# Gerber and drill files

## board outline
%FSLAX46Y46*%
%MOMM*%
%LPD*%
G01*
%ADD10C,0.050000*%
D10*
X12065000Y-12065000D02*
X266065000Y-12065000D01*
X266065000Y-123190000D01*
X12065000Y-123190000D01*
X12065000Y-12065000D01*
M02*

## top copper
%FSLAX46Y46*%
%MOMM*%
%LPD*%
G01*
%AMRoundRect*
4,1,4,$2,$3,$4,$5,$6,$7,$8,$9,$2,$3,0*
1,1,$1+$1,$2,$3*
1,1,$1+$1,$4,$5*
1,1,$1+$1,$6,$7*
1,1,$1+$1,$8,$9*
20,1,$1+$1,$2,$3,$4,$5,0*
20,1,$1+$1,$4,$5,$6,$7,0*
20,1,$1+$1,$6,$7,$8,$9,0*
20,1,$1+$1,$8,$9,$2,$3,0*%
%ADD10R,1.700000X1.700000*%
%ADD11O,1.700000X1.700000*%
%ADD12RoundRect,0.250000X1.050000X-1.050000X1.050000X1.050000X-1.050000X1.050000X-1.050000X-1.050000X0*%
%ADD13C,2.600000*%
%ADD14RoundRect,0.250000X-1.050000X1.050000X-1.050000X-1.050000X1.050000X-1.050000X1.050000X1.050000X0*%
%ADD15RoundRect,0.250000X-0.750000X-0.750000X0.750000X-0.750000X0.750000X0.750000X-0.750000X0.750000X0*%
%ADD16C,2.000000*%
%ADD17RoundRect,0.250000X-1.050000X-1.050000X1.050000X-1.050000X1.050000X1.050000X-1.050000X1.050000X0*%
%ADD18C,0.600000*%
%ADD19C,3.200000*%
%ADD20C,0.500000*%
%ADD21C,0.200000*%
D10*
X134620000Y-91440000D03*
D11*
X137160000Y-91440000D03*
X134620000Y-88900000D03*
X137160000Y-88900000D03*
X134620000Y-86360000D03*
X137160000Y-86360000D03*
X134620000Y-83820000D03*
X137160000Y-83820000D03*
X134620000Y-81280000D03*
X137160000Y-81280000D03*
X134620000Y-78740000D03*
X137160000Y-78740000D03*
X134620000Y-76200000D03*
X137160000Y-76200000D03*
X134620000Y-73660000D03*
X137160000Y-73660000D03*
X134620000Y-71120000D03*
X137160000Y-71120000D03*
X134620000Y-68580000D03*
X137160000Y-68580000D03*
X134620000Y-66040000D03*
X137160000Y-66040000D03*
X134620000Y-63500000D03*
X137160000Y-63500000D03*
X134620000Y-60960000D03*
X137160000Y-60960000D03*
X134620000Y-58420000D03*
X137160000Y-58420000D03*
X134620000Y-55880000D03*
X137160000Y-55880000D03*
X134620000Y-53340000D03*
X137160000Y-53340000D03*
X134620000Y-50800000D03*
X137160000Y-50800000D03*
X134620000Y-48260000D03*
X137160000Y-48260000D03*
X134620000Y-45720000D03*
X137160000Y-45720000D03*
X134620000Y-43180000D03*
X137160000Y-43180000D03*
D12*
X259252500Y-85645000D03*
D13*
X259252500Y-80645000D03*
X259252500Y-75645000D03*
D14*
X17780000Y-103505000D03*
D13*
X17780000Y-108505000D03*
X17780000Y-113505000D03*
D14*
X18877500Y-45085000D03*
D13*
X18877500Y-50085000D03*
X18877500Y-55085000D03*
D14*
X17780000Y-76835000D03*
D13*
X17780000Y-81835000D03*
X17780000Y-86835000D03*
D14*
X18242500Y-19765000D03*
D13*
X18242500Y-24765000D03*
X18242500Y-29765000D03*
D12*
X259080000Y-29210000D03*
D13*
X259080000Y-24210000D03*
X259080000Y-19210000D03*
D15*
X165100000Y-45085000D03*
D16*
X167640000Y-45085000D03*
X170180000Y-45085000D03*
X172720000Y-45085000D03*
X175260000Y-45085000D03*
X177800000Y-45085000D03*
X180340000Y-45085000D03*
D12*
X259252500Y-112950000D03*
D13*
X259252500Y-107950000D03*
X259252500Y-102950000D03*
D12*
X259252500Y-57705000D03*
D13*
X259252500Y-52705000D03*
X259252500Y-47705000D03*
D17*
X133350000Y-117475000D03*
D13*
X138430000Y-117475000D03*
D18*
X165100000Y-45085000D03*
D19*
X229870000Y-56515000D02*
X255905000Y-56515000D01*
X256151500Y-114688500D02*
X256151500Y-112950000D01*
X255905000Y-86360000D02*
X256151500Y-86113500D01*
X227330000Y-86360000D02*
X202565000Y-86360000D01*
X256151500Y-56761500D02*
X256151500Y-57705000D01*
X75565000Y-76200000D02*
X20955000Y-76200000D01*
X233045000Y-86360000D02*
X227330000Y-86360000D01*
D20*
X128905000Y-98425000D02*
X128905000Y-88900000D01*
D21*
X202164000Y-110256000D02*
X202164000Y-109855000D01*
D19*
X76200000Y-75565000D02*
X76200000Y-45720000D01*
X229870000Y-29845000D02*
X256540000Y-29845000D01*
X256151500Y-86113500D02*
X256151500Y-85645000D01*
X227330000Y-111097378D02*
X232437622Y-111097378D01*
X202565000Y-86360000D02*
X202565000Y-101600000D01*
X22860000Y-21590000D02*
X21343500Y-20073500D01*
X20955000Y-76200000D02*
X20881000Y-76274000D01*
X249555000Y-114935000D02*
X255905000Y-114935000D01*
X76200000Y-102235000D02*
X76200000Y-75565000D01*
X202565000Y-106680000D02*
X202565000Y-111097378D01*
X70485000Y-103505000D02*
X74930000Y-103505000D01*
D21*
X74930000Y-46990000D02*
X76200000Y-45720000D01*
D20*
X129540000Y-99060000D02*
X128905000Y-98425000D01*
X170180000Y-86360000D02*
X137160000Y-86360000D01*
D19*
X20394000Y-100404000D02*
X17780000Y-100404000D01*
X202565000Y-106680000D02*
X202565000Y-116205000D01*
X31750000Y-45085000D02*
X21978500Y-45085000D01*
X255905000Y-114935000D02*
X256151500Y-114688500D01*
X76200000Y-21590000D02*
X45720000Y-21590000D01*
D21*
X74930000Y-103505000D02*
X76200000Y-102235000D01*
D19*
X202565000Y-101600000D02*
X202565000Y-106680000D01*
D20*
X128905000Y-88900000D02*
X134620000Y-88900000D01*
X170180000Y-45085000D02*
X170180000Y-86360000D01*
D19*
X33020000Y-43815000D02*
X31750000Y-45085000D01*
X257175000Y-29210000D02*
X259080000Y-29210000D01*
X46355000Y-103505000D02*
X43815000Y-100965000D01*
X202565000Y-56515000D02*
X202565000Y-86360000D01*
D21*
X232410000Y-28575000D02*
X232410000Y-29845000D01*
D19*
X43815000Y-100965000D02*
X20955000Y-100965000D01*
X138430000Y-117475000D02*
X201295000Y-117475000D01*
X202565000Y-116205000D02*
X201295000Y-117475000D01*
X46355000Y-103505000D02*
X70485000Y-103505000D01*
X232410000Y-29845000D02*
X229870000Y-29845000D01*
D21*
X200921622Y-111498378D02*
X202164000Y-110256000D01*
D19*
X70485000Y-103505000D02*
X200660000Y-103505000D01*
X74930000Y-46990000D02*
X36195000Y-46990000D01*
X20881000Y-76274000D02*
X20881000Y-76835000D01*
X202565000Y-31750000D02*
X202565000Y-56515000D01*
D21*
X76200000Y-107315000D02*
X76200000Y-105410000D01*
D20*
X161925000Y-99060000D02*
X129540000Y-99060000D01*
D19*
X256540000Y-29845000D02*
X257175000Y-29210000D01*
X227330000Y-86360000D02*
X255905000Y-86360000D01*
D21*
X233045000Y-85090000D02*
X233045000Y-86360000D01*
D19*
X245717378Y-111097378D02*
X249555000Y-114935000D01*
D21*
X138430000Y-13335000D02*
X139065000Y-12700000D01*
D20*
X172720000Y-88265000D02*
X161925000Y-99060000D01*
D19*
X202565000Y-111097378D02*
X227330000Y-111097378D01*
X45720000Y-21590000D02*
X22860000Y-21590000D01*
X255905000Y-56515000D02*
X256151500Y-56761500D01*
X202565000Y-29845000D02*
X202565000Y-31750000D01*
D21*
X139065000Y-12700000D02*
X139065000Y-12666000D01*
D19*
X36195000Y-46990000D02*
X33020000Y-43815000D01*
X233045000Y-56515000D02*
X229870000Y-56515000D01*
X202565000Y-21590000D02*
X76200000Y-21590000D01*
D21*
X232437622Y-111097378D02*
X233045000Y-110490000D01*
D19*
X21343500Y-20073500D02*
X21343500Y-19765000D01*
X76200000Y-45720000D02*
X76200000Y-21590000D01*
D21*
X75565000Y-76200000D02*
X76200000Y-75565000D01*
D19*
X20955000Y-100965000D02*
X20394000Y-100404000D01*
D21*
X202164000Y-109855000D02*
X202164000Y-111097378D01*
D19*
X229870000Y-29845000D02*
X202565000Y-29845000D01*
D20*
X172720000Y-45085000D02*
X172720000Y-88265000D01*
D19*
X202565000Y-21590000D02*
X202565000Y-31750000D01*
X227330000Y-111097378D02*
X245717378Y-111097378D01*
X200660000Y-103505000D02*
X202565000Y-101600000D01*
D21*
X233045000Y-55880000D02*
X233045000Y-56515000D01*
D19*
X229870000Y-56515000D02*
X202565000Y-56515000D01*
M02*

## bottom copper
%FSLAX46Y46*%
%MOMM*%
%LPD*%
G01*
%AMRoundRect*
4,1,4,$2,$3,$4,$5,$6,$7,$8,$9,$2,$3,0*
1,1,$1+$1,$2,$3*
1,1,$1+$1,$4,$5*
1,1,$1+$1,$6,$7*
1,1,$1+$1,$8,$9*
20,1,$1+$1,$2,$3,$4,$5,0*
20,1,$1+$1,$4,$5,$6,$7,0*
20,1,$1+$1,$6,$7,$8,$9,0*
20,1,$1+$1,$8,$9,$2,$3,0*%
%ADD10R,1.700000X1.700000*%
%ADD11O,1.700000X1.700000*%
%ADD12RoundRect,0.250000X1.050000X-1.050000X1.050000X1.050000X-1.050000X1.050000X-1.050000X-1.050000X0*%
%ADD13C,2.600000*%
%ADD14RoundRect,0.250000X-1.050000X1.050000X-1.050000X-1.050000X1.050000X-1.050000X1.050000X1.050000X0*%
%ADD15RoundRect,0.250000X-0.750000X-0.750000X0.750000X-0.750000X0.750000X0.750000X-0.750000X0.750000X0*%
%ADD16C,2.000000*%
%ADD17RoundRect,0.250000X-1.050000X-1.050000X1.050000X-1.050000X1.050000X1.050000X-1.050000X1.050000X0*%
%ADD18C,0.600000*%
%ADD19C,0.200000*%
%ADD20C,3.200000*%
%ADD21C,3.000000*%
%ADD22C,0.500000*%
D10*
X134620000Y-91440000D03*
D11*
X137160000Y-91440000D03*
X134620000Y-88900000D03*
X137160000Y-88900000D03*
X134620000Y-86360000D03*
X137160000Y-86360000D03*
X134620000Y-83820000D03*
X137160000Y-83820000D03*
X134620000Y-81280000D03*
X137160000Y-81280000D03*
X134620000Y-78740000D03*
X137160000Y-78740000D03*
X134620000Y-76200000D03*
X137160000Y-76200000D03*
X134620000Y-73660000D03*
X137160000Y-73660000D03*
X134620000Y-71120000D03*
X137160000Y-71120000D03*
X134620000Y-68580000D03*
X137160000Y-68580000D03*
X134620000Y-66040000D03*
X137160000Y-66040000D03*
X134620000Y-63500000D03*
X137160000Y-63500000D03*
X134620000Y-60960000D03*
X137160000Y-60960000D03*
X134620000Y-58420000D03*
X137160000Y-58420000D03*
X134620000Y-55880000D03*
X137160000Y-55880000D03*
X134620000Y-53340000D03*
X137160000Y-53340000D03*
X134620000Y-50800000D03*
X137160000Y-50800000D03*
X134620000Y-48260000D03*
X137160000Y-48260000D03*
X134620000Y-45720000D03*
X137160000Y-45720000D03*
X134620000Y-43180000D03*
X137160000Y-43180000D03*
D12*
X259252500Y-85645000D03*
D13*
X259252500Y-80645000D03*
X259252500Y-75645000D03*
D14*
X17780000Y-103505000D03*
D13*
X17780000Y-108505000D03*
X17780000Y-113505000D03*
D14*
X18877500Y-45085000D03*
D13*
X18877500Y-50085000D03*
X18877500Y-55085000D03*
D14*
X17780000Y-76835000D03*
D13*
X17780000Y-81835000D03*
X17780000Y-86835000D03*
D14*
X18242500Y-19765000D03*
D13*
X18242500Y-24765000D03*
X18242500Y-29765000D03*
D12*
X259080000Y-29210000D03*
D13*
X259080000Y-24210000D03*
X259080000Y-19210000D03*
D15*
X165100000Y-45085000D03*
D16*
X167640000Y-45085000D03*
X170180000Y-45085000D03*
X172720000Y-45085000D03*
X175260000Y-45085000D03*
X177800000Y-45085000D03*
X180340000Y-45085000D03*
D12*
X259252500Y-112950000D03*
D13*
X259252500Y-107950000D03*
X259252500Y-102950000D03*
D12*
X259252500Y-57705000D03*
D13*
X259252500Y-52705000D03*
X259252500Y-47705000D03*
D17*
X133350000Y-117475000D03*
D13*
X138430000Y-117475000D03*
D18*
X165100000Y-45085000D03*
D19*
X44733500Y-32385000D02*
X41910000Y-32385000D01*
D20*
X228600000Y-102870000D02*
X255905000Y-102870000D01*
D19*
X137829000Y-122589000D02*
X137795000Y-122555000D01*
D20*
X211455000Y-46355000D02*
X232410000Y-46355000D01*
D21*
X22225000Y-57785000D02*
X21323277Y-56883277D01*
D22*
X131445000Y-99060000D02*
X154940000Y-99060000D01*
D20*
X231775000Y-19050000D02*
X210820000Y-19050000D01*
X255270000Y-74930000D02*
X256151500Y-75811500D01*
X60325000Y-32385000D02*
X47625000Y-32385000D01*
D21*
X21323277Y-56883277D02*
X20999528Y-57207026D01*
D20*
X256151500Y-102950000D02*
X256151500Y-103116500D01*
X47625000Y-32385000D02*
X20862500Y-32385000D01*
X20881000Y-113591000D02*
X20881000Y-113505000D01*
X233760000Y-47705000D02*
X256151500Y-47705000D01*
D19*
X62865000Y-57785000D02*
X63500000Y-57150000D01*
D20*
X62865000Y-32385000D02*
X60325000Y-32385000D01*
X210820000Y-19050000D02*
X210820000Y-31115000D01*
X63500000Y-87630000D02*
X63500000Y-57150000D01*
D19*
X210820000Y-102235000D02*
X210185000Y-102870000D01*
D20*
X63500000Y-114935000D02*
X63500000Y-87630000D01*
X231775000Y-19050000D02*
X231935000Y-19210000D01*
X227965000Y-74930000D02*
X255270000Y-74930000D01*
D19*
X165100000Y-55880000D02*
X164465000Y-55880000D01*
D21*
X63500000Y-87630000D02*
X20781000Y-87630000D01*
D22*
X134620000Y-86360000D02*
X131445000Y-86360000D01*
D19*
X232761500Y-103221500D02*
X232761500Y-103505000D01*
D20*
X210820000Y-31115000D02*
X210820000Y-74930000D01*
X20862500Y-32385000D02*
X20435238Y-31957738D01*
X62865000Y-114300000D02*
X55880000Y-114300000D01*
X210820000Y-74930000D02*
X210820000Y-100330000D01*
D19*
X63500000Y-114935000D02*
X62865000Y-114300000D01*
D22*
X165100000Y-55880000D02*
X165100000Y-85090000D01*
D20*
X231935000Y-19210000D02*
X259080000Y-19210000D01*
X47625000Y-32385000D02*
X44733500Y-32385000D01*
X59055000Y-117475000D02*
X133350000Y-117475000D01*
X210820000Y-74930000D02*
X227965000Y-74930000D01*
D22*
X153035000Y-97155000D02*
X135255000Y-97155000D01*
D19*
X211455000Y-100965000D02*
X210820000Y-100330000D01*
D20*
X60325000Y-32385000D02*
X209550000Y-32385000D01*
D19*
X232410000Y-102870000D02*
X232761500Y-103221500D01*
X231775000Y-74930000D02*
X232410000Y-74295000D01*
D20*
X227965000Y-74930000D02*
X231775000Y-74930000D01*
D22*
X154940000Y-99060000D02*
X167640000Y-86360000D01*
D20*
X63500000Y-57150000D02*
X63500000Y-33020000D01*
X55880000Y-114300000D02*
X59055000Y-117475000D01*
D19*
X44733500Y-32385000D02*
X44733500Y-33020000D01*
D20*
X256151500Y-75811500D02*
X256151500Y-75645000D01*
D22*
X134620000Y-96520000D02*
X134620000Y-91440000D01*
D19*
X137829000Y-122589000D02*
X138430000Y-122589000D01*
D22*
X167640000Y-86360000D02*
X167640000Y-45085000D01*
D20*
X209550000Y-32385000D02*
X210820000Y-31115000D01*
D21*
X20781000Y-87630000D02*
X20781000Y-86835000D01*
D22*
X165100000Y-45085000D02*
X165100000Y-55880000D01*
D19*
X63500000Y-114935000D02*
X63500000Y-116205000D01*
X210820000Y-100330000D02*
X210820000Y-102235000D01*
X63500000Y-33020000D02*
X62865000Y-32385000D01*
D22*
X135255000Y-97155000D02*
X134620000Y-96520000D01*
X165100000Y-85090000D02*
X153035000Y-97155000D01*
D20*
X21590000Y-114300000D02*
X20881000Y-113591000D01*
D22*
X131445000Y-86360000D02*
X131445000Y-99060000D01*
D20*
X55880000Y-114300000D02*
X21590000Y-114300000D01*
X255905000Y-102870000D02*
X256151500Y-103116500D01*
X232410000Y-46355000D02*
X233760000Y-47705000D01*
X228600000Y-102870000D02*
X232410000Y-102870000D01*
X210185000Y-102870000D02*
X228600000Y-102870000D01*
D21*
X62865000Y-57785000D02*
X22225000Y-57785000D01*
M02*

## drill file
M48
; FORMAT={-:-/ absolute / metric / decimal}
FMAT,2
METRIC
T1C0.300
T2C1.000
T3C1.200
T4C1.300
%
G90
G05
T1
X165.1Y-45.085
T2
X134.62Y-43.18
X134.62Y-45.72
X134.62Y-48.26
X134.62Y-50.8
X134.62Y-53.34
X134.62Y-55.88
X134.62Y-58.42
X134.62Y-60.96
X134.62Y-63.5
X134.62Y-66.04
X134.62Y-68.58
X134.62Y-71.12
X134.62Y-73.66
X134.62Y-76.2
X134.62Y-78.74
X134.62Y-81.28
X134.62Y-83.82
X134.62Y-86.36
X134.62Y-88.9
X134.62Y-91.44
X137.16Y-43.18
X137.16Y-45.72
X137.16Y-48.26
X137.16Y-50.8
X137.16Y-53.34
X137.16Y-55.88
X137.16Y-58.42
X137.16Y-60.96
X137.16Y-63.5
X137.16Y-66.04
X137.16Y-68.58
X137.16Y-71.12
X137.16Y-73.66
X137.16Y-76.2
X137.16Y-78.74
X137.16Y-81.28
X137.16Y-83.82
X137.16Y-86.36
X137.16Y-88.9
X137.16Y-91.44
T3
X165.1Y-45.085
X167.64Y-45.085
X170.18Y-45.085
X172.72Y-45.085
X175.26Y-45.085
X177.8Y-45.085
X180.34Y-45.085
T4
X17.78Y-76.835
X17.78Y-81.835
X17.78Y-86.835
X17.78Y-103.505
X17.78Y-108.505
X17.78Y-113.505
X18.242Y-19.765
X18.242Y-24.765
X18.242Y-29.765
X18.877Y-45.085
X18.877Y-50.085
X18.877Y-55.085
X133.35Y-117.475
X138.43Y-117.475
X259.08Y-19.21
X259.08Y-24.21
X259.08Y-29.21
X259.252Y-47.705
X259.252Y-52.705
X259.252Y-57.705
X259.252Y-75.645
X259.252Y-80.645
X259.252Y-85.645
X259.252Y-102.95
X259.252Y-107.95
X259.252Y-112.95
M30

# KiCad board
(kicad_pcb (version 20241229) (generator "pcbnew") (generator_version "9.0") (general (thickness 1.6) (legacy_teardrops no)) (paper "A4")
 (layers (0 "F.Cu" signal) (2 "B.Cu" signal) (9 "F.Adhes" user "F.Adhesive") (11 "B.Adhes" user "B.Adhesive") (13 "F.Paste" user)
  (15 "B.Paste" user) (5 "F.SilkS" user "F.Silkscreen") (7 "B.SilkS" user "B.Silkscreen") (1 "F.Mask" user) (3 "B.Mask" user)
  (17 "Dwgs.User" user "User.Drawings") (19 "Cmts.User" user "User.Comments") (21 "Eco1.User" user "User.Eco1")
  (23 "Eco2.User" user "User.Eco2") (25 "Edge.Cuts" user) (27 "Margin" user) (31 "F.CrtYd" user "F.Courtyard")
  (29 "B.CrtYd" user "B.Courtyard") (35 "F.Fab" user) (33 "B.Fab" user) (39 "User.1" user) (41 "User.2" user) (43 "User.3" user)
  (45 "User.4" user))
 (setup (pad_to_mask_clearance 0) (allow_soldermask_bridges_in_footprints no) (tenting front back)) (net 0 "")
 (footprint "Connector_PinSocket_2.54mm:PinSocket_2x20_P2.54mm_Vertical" (layer "F.Cu") (at 134.62 91.44 180)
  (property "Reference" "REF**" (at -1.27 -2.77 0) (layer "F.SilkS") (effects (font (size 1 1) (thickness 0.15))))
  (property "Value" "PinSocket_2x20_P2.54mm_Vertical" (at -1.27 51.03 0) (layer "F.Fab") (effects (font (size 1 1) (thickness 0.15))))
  (pad "1" thru_hole rect (at 0 0 180) (size 1.7 1.7) (drill 1) (layers "*.Cu" "*.Mask") (remove_unused_layers no))
  (pad "2" thru_hole oval (at -2.54 0 180) (size 1.7 1.7) (drill 1) (layers "*.Cu" "*.Mask") (remove_unused_layers no))
  (pad "3" thru_hole oval (at 0 2.54 180) (size 1.7 1.7) (drill 1) (layers "*.Cu" "*.Mask") (remove_unused_layers no))
  (pad "4" thru_hole oval (at -2.54 2.54 180) (size 1.7 1.7) (drill 1) (layers "*.Cu" "*.Mask") (remove_unused_layers no))
  (pad "5" thru_hole oval (at 0 5.08 180) (size 1.7 1.7) (drill 1) (layers "*.Cu" "*.Mask") (remove_unused_layers no))
  (pad "6" thru_hole oval (at -2.54 5.08 180) (size 1.7 1.7) (drill 1) (layers "*.Cu" "*.Mask") (remove_unused_layers no))
  (pad "7" thru_hole oval (at 0 7.62 180) (size 1.7 1.7) (drill 1) (layers "*.Cu" "*.Mask") (remove_unused_layers no))
  (pad "8" thru_hole oval (at -2.54 7.62 180) (size 1.7 1.7) (drill 1) (layers "*.Cu" "*.Mask") (remove_unused_layers no))
  (pad "9" thru_hole oval (at 0 10.16 180) (size 1.7 1.7) (drill 1) (layers "*.Cu" "*.Mask") (remove_unused_layers no))
  (pad "10" thru_hole oval (at -2.54 10.16 180) (size 1.7 1.7) (drill 1) (layers "*.Cu" "*.Mask") (remove_unused_layers no))
  (pad "11" thru_hole oval (at 0 12.7 180) (size 1.7 1.7) (drill 1) (layers "*.Cu" "*.Mask") (remove_unused_layers no))
  (pad "12" thru_hole oval (at -2.54 12.7 180) (size 1.7 1.7) (drill 1) (layers "*.Cu" "*.Mask") (remove_unused_layers no))
  (pad "13" thru_hole oval (at 0 15.24 180) (size 1.7 1.7) (drill 1) (layers "*.Cu" "*.Mask") (remove_unused_layers no))
  (pad "14" thru_hole oval (at -2.54 15.24 180) (size 1.7 1.7) (drill 1) (layers "*.Cu" "*.Mask") (remove_unused_layers no))
  (pad "15" thru_hole oval (at 0 17.78 180) (size 1.7 1.7) (drill 1) (layers "*.Cu" "*.Mask") (remove_unused_layers no))
  (pad "16" thru_hole oval (at -2.54 17.78 180) (size 1.7 1.7) (drill 1) (layers "*.Cu" "*.Mask") (remove_unused_layers no))
  (pad "17" thru_hole oval (at 0 20.32 180) (size 1.7 1.7) (drill 1) (layers "*.Cu" "*.Mask") (remove_unused_layers no))
  (pad "18" thru_hole oval (at -2.54 20.32 180) (size 1.7 1.7) (drill 1) (layers "*.Cu" "*.Mask") (remove_unused_layers no))
  (pad "19" thru_hole oval (at 0 22.86 180) (size 1.7 1.7) (drill 1) (layers "*.Cu" "*.Mask") (remove_unused_layers no))
  (pad "20" thru_hole oval (at -2.54 22.86 180) (size 1.7 1.7) (drill 1) (layers "*.Cu" "*.Mask") (remove_unused_layers no))
  (pad "21" thru_hole oval (at 0 25.4 180) (size 1.7 1.7) (drill 1) (layers "*.Cu" "*.Mask") (remove_unused_layers no))
  (pad "22" thru_hole oval (at -2.54 25.4 180) (size 1.7 1.7) (drill 1) (layers "*.Cu" "*.Mask") (remove_unused_layers no))
  (pad "23" thru_hole oval (at 0 27.94 180) (size 1.7 1.7) (drill 1) (layers "*.Cu" "*.Mask") (remove_unused_layers no))
  (pad "24" thru_hole oval (at -2.54 27.94 180) (size 1.7 1.7) (drill 1) (layers "*.Cu" "*.Mask") (remove_unused_layers no))
  (pad "25" thru_hole oval (at 0 30.48 180) (size 1.7 1.7) (drill 1) (layers "*.Cu" "*.Mask") (remove_unused_layers no))
  (pad "26" thru_hole oval (at -2.54 30.48 180) (size 1.7 1.7) (drill 1) (layers "*.Cu" "*.Mask") (remove_unused_layers no))
  (pad "27" thru_hole oval (at 0 33.02 180) (size 1.7 1.7) (drill 1) (layers "*.Cu" "*.Mask") (remove_unused_layers no))
  (pad "28" thru_hole oval (at -2.54 33.02 180) (size 1.7 1.7) (drill 1) (layers "*.Cu" "*.Mask") (remove_unused_layers no))
  (pad "29" thru_hole oval (at 0 35.56 180) (size 1.7 1.7) (drill 1) (layers "*.Cu" "*.Mask") (remove_unused_layers no))
  (pad "30" thru_hole oval (at -2.54 35.56 180) (size 1.7 1.7) (drill 1) (layers "*.Cu" "*.Mask") (remove_unused_layers no))
  (pad "31" thru_hole oval (at 0 38.1 180) (size 1.7 1.7) (drill 1) (layers "*.Cu" "*.Mask") (remove_unused_layers no))
  (pad "32" thru_hole oval (at -2.54 38.1 180) (size 1.7 1.7) (drill 1) (layers "*.Cu" "*.Mask") (remove_unused_layers no))
  (pad "33" thru_hole oval (at 0 40.64 180) (size 1.7 1.7) (drill 1) (layers "*.Cu" "*.Mask") (remove_unused_layers no))
  (pad "34" thru_hole oval (at -2.54 40.64 180) (size 1.7 1.7) (drill 1) (layers "*.Cu" "*.Mask") (remove_unused_layers no))
  (pad "35" thru_hole oval (at 0 43.18 180) (size 1.7 1.7) (drill 1) (layers "*.Cu" "*.Mask") (remove_unused_layers no))
  (pad "36" thru_hole oval (at -2.54 43.18 180) (size 1.7 1.7) (drill 1) (layers "*.Cu" "*.Mask") (remove_unused_layers no))
  (pad "37" thru_hole oval (at 0 45.72 180) (size 1.7 1.7) (drill 1) (layers "*.Cu" "*.Mask") (remove_unused_layers no))
  (pad "38" thru_hole oval (at -2.54 45.72 180) (size 1.7 1.7) (drill 1) (layers "*.Cu" "*.Mask") (remove_unused_layers no))
  (pad "39" thru_hole oval (at 0 48.26 180) (size 1.7 1.7) (drill 1) (layers "*.Cu" "*.Mask") (remove_unused_layers no))
  (pad "40" thru_hole oval (at -2.54 48.26 180) (size 1.7 1.7) (drill 1) (layers "*.Cu" "*.Mask") (remove_unused_layers no)))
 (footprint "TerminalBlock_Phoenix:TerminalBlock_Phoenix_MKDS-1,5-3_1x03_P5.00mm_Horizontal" (layer "F.Cu") (at 259.2525 85.645 90)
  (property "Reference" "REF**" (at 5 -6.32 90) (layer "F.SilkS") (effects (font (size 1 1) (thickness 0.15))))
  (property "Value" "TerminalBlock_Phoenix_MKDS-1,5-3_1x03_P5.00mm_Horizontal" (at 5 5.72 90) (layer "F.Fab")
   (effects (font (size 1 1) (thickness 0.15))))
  (pad "1" thru_hole roundrect (at 0 0 90) (size 2.6 2.6) (drill 1.3) (layers "*.Cu" "*.Mask") (remove_unused_layers no)
   (roundrect_rratio 0.096154))
  (pad "2" thru_hole circle (at 5 0 90) (size 2.6 2.6) (drill 1.3) (layers "*.Cu" "*.Mask") (remove_unused_layers no))
  (pad "3" thru_hole circle (at 10 0 90) (size 2.6 2.6) (drill 1.3) (layers "*.Cu" "*.Mask") (remove_unused_layers no)))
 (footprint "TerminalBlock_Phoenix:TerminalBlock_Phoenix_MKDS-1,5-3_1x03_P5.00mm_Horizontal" (layer "F.Cu") (at 17.78 103.505 -90)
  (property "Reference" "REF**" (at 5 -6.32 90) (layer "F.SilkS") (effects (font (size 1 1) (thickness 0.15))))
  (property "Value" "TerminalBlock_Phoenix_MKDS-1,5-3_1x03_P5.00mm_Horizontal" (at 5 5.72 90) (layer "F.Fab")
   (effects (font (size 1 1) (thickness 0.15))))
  (pad "1" thru_hole roundrect (at 0 0 270) (size 2.6 2.6) (drill 1.3) (layers "*.Cu" "*.Mask") (remove_unused_layers no)
   (roundrect_rratio 0.096154))
  (pad "2" thru_hole circle (at 5 0 270) (size 2.6 2.6) (drill 1.3) (layers "*.Cu" "*.Mask") (remove_unused_layers no))
  (pad "3" thru_hole circle (at 10 0 270) (size 2.6 2.6) (drill 1.3) (layers "*.Cu" "*.Mask") (remove_unused_layers no)))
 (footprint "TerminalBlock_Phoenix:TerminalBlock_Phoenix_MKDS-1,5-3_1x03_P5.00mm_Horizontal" (layer "F.Cu") (at 18.8775 45.085 -90)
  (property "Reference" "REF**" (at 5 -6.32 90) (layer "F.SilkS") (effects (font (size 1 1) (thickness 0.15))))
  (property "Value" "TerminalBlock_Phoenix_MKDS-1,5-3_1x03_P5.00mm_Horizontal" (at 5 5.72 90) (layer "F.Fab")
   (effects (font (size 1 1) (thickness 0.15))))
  (pad "1" thru_hole roundrect (at 0 0 270) (size 2.6 2.6) (drill 1.3) (layers "*.Cu" "*.Mask") (remove_unused_layers no)
   (roundrect_rratio 0.096154))
  (pad "2" thru_hole circle (at 5 0 270) (size 2.6 2.6) (drill 1.3) (layers "*.Cu" "*.Mask") (remove_unused_layers no))
  (pad "3" thru_hole circle (at 10 0 270) (size 2.6 2.6) (drill 1.3) (layers "*.Cu" "*.Mask") (remove_unused_layers no)))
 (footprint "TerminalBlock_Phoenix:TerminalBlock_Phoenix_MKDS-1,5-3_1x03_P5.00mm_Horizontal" (layer "F.Cu") (at 17.78 76.835 -90)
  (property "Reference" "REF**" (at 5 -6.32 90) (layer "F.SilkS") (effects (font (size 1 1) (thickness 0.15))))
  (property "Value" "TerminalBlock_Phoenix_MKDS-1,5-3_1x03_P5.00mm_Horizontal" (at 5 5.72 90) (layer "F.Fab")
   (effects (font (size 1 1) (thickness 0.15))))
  (pad "1" thru_hole roundrect (at 0 0 270) (size 2.6 2.6) (drill 1.3) (layers "*.Cu" "*.Mask") (remove_unused_layers no)
   (roundrect_rratio 0.096154))
  (pad "2" thru_hole circle (at 5 0 270) (size 2.6 2.6) (drill 1.3) (layers "*.Cu" "*.Mask") (remove_unused_layers no))
  (pad "3" thru_hole circle (at 10 0 270) (size 2.6 2.6) (drill 1.3) (layers "*.Cu" "*.Mask") (remove_unused_layers no)))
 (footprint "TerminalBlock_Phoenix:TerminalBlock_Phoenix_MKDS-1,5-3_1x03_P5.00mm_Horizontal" (layer "F.Cu") (at 18.2425 19.765 -90)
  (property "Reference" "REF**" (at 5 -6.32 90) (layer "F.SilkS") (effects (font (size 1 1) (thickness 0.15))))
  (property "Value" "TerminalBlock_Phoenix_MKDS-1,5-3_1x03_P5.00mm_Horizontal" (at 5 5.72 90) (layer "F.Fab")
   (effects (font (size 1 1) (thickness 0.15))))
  (pad "1" thru_hole roundrect (at 0 0 270) (size 2.6 2.6) (drill 1.3) (layers "*.Cu" "*.Mask") (remove_unused_layers no)
   (roundrect_rratio 0.096154))
  (pad "2" thru_hole circle (at 5 0 270) (size 2.6 2.6) (drill 1.3) (layers "*.Cu" "*.Mask") (remove_unused_layers no))
  (pad "3" thru_hole circle (at 10 0 270) (size 2.6 2.6) (drill 1.3) (layers "*.Cu" "*.Mask") (remove_unused_layers no)))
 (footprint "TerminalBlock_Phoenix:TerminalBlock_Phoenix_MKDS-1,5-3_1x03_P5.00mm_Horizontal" (layer "F.Cu") (at 259.08 29.21 90)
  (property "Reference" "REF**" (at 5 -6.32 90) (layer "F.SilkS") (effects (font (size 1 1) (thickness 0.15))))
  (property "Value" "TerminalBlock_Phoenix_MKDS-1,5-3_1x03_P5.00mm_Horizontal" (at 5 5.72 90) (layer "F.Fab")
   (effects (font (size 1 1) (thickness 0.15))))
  (pad "1" thru_hole roundrect (at 0 0 90) (size 2.6 2.6) (drill 1.3) (layers "*.Cu" "*.Mask") (remove_unused_layers no)
   (roundrect_rratio 0.096154))
  (pad "2" thru_hole circle (at 5 0 90) (size 2.6 2.6) (drill 1.3) (layers "*.Cu" "*.Mask") (remove_unused_layers no))
  (pad "3" thru_hole circle (at 10 0 90) (size 2.6 2.6) (drill 1.3) (layers "*.Cu" "*.Mask") (remove_unused_layers no)))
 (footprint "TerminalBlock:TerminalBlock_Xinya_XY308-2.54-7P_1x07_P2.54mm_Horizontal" (layer "F.Cu") (at 165.1 45.085)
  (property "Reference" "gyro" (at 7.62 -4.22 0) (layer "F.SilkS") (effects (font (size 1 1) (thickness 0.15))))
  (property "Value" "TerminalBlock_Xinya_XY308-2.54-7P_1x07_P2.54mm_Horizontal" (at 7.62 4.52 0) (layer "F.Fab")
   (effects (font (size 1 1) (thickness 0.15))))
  (pad "1" thru_hole roundrect (at 0 0) (size 2 2) (drill 1.2) (layers "*.Cu" "*.Mask") (remove_unused_layers no) (roundrect_rratio 0.125))
  (pad "2" thru_hole circle (at 2.54 0) (size 2 2) (drill 1.2) (layers "*.Cu" "*.Mask") (remove_unused_layers no))
  (pad "3" thru_hole circle (at 5.08 0) (size 2 2) (drill 1.2) (layers "*.Cu" "*.Mask") (remove_unused_layers no))
  (pad "4" thru_hole circle (at 7.62 0) (size 2 2) (drill 1.2) (layers "*.Cu" "*.Mask") (remove_unused_layers no))
  (pad "5" thru_hole circle (at 10.16 0) (size 2 2) (drill 1.2) (layers "*.Cu" "*.Mask") (remove_unused_layers no))
  (pad "6" thru_hole circle (at 12.7 0) (size 2 2) (drill 1.2) (layers "*.Cu" "*.Mask") (remove_unused_layers no))
  (pad "7" thru_hole circle (at 15.24 0) (size 2 2) (drill 1.2) (layers "*.Cu" "*.Mask") (remove_unused_layers no)))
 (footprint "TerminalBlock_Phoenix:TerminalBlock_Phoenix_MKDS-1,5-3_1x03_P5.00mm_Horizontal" (layer "F.Cu") (at 259.2525 112.95 90)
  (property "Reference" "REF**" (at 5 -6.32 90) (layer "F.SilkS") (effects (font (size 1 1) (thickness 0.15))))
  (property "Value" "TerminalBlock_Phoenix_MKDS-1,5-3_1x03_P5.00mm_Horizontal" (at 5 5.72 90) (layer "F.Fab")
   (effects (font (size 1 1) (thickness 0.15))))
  (pad "1" thru_hole roundrect (at 0 0 90) (size 2.6 2.6) (drill 1.3) (layers "*.Cu" "*.Mask") (remove_unused_layers no)
   (roundrect_rratio 0.096154))
  (pad "2" thru_hole circle (at 5 0 90) (size 2.6 2.6) (drill 1.3) (layers "*.Cu" "*.Mask") (remove_unused_layers no))
  (pad "3" thru_hole circle (at 10 0 90) (size 2.6 2.6) (drill 1.3) (layers "*.Cu" "*.Mask") (remove_unused_layers no)))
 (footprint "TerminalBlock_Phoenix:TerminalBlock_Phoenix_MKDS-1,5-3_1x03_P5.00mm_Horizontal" (layer "F.Cu") (at 259.2525 57.705 90)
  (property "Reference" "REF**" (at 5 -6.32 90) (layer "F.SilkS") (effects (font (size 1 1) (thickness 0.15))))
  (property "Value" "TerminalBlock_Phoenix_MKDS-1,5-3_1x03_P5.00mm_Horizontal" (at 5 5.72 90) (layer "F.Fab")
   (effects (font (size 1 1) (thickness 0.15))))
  (pad "1" thru_hole roundrect (at 0 0 90) (size 2.6 2.6) (drill 1.3) (layers "*.Cu" "*.Mask") (remove_unused_layers no)
   (roundrect_rratio 0.096154))
  (pad "2" thru_hole circle (at 5 0 90) (size 2.6 2.6) (drill 1.3) (layers "*.Cu" "*.Mask") (remove_unused_layers no))
  (pad "3" thru_hole circle (at 10 0 90) (size 2.6 2.6) (drill 1.3) (layers "*.Cu" "*.Mask") (remove_unused_layers no)))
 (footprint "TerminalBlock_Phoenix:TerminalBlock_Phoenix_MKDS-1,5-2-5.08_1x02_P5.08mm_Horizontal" (layer "F.Cu") (at 133.35 117.475)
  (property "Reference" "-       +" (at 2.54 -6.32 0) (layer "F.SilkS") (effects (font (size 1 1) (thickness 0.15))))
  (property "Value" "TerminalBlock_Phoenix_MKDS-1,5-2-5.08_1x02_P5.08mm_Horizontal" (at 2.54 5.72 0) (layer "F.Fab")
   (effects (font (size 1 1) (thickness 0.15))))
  (pad "1" thru_hole roundrect (at 0 0) (size 2.6 2.6) (drill 1.3) (layers "*.Cu" "*.Mask") (remove_unused_layers no)
   (roundrect_rratio 0.096154))
  (pad "2" thru_hole circle (at 5.08 0) (size 2.6 2.6) (drill 1.3) (layers "*.Cu" "*.Mask") (remove_unused_layers no)))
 (gr_rect (start 12.065 12.065) (end 266.065 123.19) (stroke (width 0.05) (type default)) (fill no) (layer "Edge.Cuts"))
 (segment (start 229.87 56.515) (end 255.905 56.515) (width 3.2) (layer "F.Cu") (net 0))
 (segment (start 256.1515 114.6885) (end 256.1515 112.95) (width 3.2) (layer "F.Cu") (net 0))
 (segment (start 255.905 86.36) (end 256.1515 86.1135) (width 3.2) (layer "F.Cu") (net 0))
 (segment (start 227.33 86.36) (end 202.565 86.36) (width 3.2) (layer "F.Cu") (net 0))
 (segment (start 256.1515 56.7615) (end 256.1515 57.705) (width 3.2) (layer "F.Cu") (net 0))
 (segment (start 75.565 76.2) (end 20.955 76.2) (width 3.2) (layer "F.Cu") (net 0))
 (segment (start 233.045 86.36) (end 227.33 86.36) (width 3.2) (layer "F.Cu") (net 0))
 (segment (start 128.905 98.425) (end 128.905 88.9) (width 0.5) (layer "F.Cu") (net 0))
 (segment (start 202.164 110.256) (end 202.164 109.855) (width 0.2) (layer "F.Cu") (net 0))
 (segment (start 76.2 75.565) (end 76.2 45.72) (width 3.2) (layer "F.Cu") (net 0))
 (segment (start 229.87 29.845) (end 256.54 29.845) (width 3.2) (layer "F.Cu") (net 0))
 (segment (start 256.1515 86.1135) (end 256.1515 85.645) (width 3.2) (layer "F.Cu") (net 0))
 (segment (start 227.33 111.097378) (end 232.437622 111.097378) (width 3.2) (layer "F.Cu") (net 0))
 (segment (start 202.565 86.36) (end 202.565 101.6) (width 3.2) (layer "F.Cu") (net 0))
 (segment (start 22.86 21.59) (end 21.3435 20.0735) (width 3.2) (layer "F.Cu") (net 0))
 (segment (start 20.955 76.2) (end 20.881 76.274) (width 3.2) (layer "F.Cu") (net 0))
 (segment (start 249.555 114.935) (end 255.905 114.935) (width 3.2) (layer "F.Cu") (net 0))
 (segment (start 76.2 102.235) (end 76.2 75.565) (width 3.2) (layer "F.Cu") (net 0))
 (segment (start 202.565 106.68) (end 202.565 111.097378) (width 3.2) (layer "F.Cu") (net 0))
 (segment (start 70.485 103.505) (end 74.93 103.505) (width 3.2) (layer "F.Cu") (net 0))
 (segment (start 74.93 46.99) (end 76.2 45.72) (width 0.2) (layer "F.Cu") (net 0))
 (segment (start 129.54 99.06) (end 128.905 98.425) (width 0.5) (layer "F.Cu") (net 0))
 (segment (start 170.18 86.36) (end 137.16 86.36) (width 0.5) (layer "F.Cu") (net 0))
 (segment (start 20.394 100.404) (end 17.78 100.404) (width 3.2) (layer "F.Cu") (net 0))
 (segment (start 202.565 106.68) (end 202.565 116.205) (width 3.2) (layer "F.Cu") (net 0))
 (segment (start 31.75 45.085) (end 21.9785 45.085) (width 3.2) (layer "F.Cu") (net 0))
 (segment (start 255.905 114.935) (end 256.1515 114.6885) (width 3.2) (layer "F.Cu") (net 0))
 (segment (start 76.2 21.59) (end 45.72 21.59) (width 3.2) (layer "F.Cu") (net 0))
 (segment (start 74.93 103.505) (end 76.2 102.235) (width 0.2) (layer "F.Cu") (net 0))
 (segment (start 202.565 101.6) (end 202.565 106.68) (width 3.2) (layer "F.Cu") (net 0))
 (segment (start 128.905 88.9) (end 134.62 88.9) (width 0.5) (layer "F.Cu") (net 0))
 (segment (start 170.18 45.085) (end 170.18 86.36) (width 0.5) (layer "F.Cu") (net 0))
 (segment (start 33.02 43.815) (end 31.75 45.085) (width 3.2) (layer "F.Cu") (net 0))
 (segment (start 257.175 29.21) (end 259.08 29.21) (width 3.2) (layer "F.Cu") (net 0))
 (segment (start 46.355 103.505) (end 43.815 100.965) (width 3.2) (layer "F.Cu") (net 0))
 (segment (start 202.565 56.515) (end 202.565 86.36) (width 3.2) (layer "F.Cu") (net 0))
 (segment (start 232.41 28.575) (end 232.41 29.845) (width 0.2) (layer "F.Cu") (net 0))
 (segment (start 43.815 100.965) (end 20.955 100.965) (width 3.2) (layer "F.Cu") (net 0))
 (segment (start 138.43 117.475) (end 201.295 117.475) (width 3.2) (layer "F.Cu") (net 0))
 (segment (start 202.565 116.205) (end 201.295 117.475) (width 3.2) (layer "F.Cu") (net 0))
 (segment (start 46.355 103.505) (end 70.485 103.505) (width 3.2) (layer "F.Cu") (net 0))
 (segment (start 232.41 29.845) (end 229.87 29.845) (width 3.2) (layer "F.Cu") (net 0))
 (segment (start 200.921622 111.498378) (end 202.164 110.256) (width 0.2) (layer "F.Cu") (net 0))
 (segment (start 70.485 103.505) (end 200.66 103.505) (width 3.2) (layer "F.Cu") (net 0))
 (segment (start 74.93 46.99) (end 36.195 46.99) (width 3.2) (layer "F.Cu") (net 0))
 (segment (start 20.881 76.274) (end 20.881 76.835) (width 3.2) (layer "F.Cu") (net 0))
 (segment (start 202.565 31.75) (end 202.565 56.515) (width 3.2) (layer "F.Cu") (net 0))
 (segment (start 76.2 107.315) (end 76.2 105.41) (width 0.2) (layer "F.Cu") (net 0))
 (segment (start 161.925 99.06) (end 129.54 99.06) (width 0.5) (layer "F.Cu") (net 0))
 (segment (start 256.54 29.845) (end 257.175 29.21) (width 3.2) (layer "F.Cu") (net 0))
 (segment (start 227.33 86.36) (end 255.905 86.36) (width 3.2) (layer "F.Cu") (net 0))
 (segment (start 233.045 85.09) (end 233.045 86.36) (width 0.2) (layer "F.Cu") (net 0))
 (segment (start 245.717378 111.097378) (end 249.555 114.935) (width 3.2) (layer "F.Cu") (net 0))
 (segment (start 138.43 13.335) (end 139.065 12.7) (width 0.2) (layer "F.Cu") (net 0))
 (segment (start 172.72 88.265) (end 161.925 99.06) (width 0.5) (layer "F.Cu") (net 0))
 (segment (start 202.565 111.097378) (end 227.33 111.097378) (width 3.2) (layer "F.Cu") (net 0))
 (segment (start 45.72 21.59) (end 22.86 21.59) (width 3.2) (layer "F.Cu") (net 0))
 (segment (start 255.905 56.515) (end 256.1515 56.7615) (width 3.2) (layer "F.Cu") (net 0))
 (segment (start 202.565 29.845) (end 202.565 31.75) (width 3.2) (layer "F.Cu") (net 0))
 (segment (start 139.065 12.7) (end 139.065 12.666) (width 0.2) (layer "F.Cu") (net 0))
 (segment (start 36.195 46.99) (end 33.02 43.815) (width 3.2) (layer "F.Cu") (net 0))
 (segment (start 233.045 56.515) (end 229.87 56.515) (width 3.2) (layer "F.Cu") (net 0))
 (segment (start 202.565 21.59) (end 76.2 21.59) (width 3.2) (layer "F.Cu") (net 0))
 (segment (start 232.437622 111.097378) (end 233.045 110.49) (width 0.2) (layer "F.Cu") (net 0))
 (segment (start 21.3435 20.0735) (end 21.3435 19.765) (width 3.2) (layer "F.Cu") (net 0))
 (segment (start 76.2 45.72) (end 76.2 21.59) (width 3.2) (layer "F.Cu") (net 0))
 (segment (start 75.565 76.2) (end 76.2 75.565) (width 0.2) (layer "F.Cu") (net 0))
 (segment (start 20.955 100.965) (end 20.394 100.404) (width 3.2) (layer "F.Cu") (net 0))
 (segment (start 202.164 109.855) (end 202.164 111.097378) (width 0.2) (layer "F.Cu") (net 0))
 (segment (start 229.87 29.845) (end 202.565 29.845) (width 3.2) (layer "F.Cu") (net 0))
 (segment (start 172.72 45.085) (end 172.72 88.265) (width 0.5) (layer "F.Cu") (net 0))
 (segment (start 202.565 21.59) (end 202.565 31.75) (width 3.2) (layer "F.Cu") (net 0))
 (segment (start 227.33 111.097378) (end 245.717378 111.097378) (width 3.2) (layer "F.Cu") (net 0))
 (segment (start 200.66 103.505) (end 202.565 101.6) (width 3.2) (layer "F.Cu") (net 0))
 (segment (start 233.045 55.88) (end 233.045 56.515) (width 0.2) (layer "F.Cu") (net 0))
 (segment (start 229.87 56.515) (end 202.565 56.515) (width 3.2) (layer "F.Cu") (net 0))
 (via (at 165.1 45.085) (size 0.6) (drill 0.3) (layers "F.Cu" "B.Cu") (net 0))
 (segment (start 44.7335 32.385) (end 41.91 32.385) (width 0.2) (layer "B.Cu") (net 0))
 (segment (start 228.6 102.87) (end 255.905 102.87) (width 3.2) (layer "B.Cu") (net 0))
 (segment (start 137.829 122.589) (end 137.795 122.555) (width 0.2) (layer "B.Cu") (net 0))
 (segment (start 211.455 46.355) (end 232.41 46.355) (width 3.2) (layer "B.Cu") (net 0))
 (segment (start 22.225 57.785) (end 21.323277 56.883277) (width 3) (layer "B.Cu") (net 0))
 (segment (start 131.445 99.06) (end 154.94 99.06) (width 0.5) (layer "B.Cu") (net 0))
 (segment (start 231.775 19.05) (end 210.82 19.05) (width 3.2) (layer "B.Cu") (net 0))
 (segment (start 255.27 74.93) (end 256.1515 75.8115) (width 3.2) (layer "B.Cu") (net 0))
 (segment (start 60.325 32.385) (end 47.625 32.385) (width 3.2) (layer "B.Cu") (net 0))
 (segment (start 21.323277 56.883277) (end 20.999528 57.207026) (width 3) (layer "B.Cu") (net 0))
 (segment (start 256.1515 102.95) (end 256.1515 103.1165) (width 3.2) (layer "B.Cu") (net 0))
 (segment (start 47.625 32.385) (end 20.8625 32.385) (width 3.2) (layer "B.Cu") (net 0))
 (segment (start 20.881 113.591) (end 20.881 113.505) (width 3.2) (layer "B.Cu") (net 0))
 (segment (start 233.76 47.705) (end 256.1515 47.705) (width 3.2) (layer "B.Cu") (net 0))
 (segment (start 62.865 57.785) (end 63.5 57.15) (width 0.2) (layer "B.Cu") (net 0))
 (segment (start 62.865 32.385) (end 60.325 32.385) (width 3.2) (layer "B.Cu") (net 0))
 (segment (start 210.82 19.05) (end 210.82 31.115) (width 3.2) (layer "B.Cu") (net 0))
 (segment (start 63.5 87.63) (end 63.5 57.15) (width 3.2) (layer "B.Cu") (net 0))
 (segment (start 210.82 102.235) (end 210.185 102.87) (width 0.2) (layer "B.Cu") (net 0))
 (segment (start 63.5 114.935) (end 63.5 87.63) (width 3.2) (layer "B.Cu") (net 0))
 (segment (start 231.775 19.05) (end 231.935 19.21) (width 3.2) (layer "B.Cu") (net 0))
 (segment (start 227.965 74.93) (end 255.27 74.93) (width 3.2) (layer "B.Cu") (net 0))
 (segment (start 165.1 55.88) (end 164.465 55.88) (width 0.2) (layer "B.Cu") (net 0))
 (segment (start 63.5 87.63) (end 20.781 87.63) (width 3) (layer "B.Cu") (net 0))
 (segment (start 134.62 86.36) (end 131.445 86.36) (width 0.5) (layer "B.Cu") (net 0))
 (segment (start 232.7615 103.2215) (end 232.7615 103.505) (width 0.2) (layer "B.Cu") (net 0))
 (segment (start 210.82 31.115) (end 210.82 74.93) (width 3.2) (layer "B.Cu") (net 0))
 (segment (start 20.8625 32.385) (end 20.435238 31.957738) (width 3.2) (layer "B.Cu") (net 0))
 (segment (start 62.865 114.3) (end 55.88 114.3) (width 3.2) (layer "B.Cu") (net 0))
 (segment (start 210.82 74.93) (end 210.82 100.33) (width 3.2) (layer "B.Cu") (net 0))
 (segment (start 63.5 114.935) (end 62.865 114.3) (width 0.2) (layer "B.Cu") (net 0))
 (segment (start 165.1 55.88) (end 165.1 85.09) (width 0.5) (layer "B.Cu") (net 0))
 (segment (start 231.935 19.21) (end 259.08 19.21) (width 3.2) (layer "B.Cu") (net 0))
 (segment (start 47.625 32.385) (end 44.7335 32.385) (width 3.2) (layer "B.Cu") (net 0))
 (segment (start 59.055 117.475) (end 133.35 117.475) (width 3.2) (layer "B.Cu") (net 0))
 (segment (start 210.82 74.93) (end 227.965 74.93) (width 3.2) (layer "B.Cu") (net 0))
 (segment (start 153.035 97.155) (end 135.255 97.155) (width 0.5) (layer "B.Cu") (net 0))
 (segment (start 211.455 100.965) (end 210.82 100.33) (width 0.2) (layer "B.Cu") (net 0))
 (segment (start 60.325 32.385) (end 209.55 32.385) (width 3.2) (layer "B.Cu") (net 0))
 (segment (start 232.41 102.87) (end 232.7615 103.2215) (width 0.2) (layer "B.Cu") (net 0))
 (segment (start 231.775 74.93) (end 232.41 74.295) (width 0.2) (layer "B.Cu") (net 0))
 (segment (start 227.965 74.93) (end 231.775 74.93) (width 3.2) (layer "B.Cu") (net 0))
 (segment (start 154.94 99.06) (end 167.64 86.36) (width 0.5) (layer "B.Cu") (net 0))
 (segment (start 63.5 57.15) (end 63.5 33.02) (width 3.2) (layer "B.Cu") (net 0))
 (segment (start 55.88 114.3) (end 59.055 117.475) (width 3.2) (layer "B.Cu") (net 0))
 (segment (start 44.7335 32.385) (end 44.7335 33.02) (width 0.2) (layer "B.Cu") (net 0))
 (segment (start 256.1515 75.8115) (end 256.1515 75.645) (width 3.2) (layer "B.Cu") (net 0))
 (segment (start 134.62 96.52) (end 134.62 91.44) (width 0.5) (layer "B.Cu") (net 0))
 (segment (start 137.829 122.589) (end 138.43 122.589) (width 0.2) (layer "B.Cu") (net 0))
 (segment (start 167.64 86.36) (end 167.64 45.085) (width 0.5) (layer "B.Cu") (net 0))
 (segment (start 209.55 32.385) (end 210.82 31.115) (width 3.2) (layer "B.Cu") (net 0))
 (segment (start 20.781 87.63) (end 20.781 86.835) (width 3) (layer "B.Cu") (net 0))
 (segment (start 165.1 45.085) (end 165.1 55.88) (width 0.5) (layer "B.Cu") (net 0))
 (segment (start 63.5 114.935) (end 63.5 116.205) (width 0.2) (layer "B.Cu") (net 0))
 (segment (start 210.82 100.33) (end 210.82 102.235) (width 0.2) (layer "B.Cu") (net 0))
 (segment (start 63.5 33.02) (end 62.865 32.385) (width 0.2) (layer "B.Cu") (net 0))
 (segment (start 135.255 97.155) (end 134.62 96.52) (width 0.5) (layer "B.Cu") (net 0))
 (segment (start 165.1 85.09) (end 153.035 97.155) (width 0.5) (layer "B.Cu") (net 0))
 (segment (start 21.59 114.3) (end 20.881 113.591) (width 3.2) (layer "B.Cu") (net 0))
 (segment (start 131.445 86.36) (end 131.445 99.06) (width 0.5) (layer "B.Cu") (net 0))
 (segment (start 55.88 114.3) (end 21.59 114.3) (width 3.2) (layer "B.Cu") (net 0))
 (segment (start 255.905 102.87) (end 256.1515 103.1165) (width 3.2) (layer "B.Cu") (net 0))
 (segment (start 232.41 46.355) (end 233.76 47.705) (width 3.2) (layer "B.Cu") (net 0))
 (segment (start 228.6 102.87) (end 232.41 102.87) (width 3.2) (layer "B.Cu") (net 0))
 (segment (start 210.185 102.87) (end 228.6 102.87) (width 3.2) (layer "B.Cu") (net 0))
 (segment (start 62.865 57.785) (end 22.225 57.785) (width 3) (layer "B.Cu") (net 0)))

